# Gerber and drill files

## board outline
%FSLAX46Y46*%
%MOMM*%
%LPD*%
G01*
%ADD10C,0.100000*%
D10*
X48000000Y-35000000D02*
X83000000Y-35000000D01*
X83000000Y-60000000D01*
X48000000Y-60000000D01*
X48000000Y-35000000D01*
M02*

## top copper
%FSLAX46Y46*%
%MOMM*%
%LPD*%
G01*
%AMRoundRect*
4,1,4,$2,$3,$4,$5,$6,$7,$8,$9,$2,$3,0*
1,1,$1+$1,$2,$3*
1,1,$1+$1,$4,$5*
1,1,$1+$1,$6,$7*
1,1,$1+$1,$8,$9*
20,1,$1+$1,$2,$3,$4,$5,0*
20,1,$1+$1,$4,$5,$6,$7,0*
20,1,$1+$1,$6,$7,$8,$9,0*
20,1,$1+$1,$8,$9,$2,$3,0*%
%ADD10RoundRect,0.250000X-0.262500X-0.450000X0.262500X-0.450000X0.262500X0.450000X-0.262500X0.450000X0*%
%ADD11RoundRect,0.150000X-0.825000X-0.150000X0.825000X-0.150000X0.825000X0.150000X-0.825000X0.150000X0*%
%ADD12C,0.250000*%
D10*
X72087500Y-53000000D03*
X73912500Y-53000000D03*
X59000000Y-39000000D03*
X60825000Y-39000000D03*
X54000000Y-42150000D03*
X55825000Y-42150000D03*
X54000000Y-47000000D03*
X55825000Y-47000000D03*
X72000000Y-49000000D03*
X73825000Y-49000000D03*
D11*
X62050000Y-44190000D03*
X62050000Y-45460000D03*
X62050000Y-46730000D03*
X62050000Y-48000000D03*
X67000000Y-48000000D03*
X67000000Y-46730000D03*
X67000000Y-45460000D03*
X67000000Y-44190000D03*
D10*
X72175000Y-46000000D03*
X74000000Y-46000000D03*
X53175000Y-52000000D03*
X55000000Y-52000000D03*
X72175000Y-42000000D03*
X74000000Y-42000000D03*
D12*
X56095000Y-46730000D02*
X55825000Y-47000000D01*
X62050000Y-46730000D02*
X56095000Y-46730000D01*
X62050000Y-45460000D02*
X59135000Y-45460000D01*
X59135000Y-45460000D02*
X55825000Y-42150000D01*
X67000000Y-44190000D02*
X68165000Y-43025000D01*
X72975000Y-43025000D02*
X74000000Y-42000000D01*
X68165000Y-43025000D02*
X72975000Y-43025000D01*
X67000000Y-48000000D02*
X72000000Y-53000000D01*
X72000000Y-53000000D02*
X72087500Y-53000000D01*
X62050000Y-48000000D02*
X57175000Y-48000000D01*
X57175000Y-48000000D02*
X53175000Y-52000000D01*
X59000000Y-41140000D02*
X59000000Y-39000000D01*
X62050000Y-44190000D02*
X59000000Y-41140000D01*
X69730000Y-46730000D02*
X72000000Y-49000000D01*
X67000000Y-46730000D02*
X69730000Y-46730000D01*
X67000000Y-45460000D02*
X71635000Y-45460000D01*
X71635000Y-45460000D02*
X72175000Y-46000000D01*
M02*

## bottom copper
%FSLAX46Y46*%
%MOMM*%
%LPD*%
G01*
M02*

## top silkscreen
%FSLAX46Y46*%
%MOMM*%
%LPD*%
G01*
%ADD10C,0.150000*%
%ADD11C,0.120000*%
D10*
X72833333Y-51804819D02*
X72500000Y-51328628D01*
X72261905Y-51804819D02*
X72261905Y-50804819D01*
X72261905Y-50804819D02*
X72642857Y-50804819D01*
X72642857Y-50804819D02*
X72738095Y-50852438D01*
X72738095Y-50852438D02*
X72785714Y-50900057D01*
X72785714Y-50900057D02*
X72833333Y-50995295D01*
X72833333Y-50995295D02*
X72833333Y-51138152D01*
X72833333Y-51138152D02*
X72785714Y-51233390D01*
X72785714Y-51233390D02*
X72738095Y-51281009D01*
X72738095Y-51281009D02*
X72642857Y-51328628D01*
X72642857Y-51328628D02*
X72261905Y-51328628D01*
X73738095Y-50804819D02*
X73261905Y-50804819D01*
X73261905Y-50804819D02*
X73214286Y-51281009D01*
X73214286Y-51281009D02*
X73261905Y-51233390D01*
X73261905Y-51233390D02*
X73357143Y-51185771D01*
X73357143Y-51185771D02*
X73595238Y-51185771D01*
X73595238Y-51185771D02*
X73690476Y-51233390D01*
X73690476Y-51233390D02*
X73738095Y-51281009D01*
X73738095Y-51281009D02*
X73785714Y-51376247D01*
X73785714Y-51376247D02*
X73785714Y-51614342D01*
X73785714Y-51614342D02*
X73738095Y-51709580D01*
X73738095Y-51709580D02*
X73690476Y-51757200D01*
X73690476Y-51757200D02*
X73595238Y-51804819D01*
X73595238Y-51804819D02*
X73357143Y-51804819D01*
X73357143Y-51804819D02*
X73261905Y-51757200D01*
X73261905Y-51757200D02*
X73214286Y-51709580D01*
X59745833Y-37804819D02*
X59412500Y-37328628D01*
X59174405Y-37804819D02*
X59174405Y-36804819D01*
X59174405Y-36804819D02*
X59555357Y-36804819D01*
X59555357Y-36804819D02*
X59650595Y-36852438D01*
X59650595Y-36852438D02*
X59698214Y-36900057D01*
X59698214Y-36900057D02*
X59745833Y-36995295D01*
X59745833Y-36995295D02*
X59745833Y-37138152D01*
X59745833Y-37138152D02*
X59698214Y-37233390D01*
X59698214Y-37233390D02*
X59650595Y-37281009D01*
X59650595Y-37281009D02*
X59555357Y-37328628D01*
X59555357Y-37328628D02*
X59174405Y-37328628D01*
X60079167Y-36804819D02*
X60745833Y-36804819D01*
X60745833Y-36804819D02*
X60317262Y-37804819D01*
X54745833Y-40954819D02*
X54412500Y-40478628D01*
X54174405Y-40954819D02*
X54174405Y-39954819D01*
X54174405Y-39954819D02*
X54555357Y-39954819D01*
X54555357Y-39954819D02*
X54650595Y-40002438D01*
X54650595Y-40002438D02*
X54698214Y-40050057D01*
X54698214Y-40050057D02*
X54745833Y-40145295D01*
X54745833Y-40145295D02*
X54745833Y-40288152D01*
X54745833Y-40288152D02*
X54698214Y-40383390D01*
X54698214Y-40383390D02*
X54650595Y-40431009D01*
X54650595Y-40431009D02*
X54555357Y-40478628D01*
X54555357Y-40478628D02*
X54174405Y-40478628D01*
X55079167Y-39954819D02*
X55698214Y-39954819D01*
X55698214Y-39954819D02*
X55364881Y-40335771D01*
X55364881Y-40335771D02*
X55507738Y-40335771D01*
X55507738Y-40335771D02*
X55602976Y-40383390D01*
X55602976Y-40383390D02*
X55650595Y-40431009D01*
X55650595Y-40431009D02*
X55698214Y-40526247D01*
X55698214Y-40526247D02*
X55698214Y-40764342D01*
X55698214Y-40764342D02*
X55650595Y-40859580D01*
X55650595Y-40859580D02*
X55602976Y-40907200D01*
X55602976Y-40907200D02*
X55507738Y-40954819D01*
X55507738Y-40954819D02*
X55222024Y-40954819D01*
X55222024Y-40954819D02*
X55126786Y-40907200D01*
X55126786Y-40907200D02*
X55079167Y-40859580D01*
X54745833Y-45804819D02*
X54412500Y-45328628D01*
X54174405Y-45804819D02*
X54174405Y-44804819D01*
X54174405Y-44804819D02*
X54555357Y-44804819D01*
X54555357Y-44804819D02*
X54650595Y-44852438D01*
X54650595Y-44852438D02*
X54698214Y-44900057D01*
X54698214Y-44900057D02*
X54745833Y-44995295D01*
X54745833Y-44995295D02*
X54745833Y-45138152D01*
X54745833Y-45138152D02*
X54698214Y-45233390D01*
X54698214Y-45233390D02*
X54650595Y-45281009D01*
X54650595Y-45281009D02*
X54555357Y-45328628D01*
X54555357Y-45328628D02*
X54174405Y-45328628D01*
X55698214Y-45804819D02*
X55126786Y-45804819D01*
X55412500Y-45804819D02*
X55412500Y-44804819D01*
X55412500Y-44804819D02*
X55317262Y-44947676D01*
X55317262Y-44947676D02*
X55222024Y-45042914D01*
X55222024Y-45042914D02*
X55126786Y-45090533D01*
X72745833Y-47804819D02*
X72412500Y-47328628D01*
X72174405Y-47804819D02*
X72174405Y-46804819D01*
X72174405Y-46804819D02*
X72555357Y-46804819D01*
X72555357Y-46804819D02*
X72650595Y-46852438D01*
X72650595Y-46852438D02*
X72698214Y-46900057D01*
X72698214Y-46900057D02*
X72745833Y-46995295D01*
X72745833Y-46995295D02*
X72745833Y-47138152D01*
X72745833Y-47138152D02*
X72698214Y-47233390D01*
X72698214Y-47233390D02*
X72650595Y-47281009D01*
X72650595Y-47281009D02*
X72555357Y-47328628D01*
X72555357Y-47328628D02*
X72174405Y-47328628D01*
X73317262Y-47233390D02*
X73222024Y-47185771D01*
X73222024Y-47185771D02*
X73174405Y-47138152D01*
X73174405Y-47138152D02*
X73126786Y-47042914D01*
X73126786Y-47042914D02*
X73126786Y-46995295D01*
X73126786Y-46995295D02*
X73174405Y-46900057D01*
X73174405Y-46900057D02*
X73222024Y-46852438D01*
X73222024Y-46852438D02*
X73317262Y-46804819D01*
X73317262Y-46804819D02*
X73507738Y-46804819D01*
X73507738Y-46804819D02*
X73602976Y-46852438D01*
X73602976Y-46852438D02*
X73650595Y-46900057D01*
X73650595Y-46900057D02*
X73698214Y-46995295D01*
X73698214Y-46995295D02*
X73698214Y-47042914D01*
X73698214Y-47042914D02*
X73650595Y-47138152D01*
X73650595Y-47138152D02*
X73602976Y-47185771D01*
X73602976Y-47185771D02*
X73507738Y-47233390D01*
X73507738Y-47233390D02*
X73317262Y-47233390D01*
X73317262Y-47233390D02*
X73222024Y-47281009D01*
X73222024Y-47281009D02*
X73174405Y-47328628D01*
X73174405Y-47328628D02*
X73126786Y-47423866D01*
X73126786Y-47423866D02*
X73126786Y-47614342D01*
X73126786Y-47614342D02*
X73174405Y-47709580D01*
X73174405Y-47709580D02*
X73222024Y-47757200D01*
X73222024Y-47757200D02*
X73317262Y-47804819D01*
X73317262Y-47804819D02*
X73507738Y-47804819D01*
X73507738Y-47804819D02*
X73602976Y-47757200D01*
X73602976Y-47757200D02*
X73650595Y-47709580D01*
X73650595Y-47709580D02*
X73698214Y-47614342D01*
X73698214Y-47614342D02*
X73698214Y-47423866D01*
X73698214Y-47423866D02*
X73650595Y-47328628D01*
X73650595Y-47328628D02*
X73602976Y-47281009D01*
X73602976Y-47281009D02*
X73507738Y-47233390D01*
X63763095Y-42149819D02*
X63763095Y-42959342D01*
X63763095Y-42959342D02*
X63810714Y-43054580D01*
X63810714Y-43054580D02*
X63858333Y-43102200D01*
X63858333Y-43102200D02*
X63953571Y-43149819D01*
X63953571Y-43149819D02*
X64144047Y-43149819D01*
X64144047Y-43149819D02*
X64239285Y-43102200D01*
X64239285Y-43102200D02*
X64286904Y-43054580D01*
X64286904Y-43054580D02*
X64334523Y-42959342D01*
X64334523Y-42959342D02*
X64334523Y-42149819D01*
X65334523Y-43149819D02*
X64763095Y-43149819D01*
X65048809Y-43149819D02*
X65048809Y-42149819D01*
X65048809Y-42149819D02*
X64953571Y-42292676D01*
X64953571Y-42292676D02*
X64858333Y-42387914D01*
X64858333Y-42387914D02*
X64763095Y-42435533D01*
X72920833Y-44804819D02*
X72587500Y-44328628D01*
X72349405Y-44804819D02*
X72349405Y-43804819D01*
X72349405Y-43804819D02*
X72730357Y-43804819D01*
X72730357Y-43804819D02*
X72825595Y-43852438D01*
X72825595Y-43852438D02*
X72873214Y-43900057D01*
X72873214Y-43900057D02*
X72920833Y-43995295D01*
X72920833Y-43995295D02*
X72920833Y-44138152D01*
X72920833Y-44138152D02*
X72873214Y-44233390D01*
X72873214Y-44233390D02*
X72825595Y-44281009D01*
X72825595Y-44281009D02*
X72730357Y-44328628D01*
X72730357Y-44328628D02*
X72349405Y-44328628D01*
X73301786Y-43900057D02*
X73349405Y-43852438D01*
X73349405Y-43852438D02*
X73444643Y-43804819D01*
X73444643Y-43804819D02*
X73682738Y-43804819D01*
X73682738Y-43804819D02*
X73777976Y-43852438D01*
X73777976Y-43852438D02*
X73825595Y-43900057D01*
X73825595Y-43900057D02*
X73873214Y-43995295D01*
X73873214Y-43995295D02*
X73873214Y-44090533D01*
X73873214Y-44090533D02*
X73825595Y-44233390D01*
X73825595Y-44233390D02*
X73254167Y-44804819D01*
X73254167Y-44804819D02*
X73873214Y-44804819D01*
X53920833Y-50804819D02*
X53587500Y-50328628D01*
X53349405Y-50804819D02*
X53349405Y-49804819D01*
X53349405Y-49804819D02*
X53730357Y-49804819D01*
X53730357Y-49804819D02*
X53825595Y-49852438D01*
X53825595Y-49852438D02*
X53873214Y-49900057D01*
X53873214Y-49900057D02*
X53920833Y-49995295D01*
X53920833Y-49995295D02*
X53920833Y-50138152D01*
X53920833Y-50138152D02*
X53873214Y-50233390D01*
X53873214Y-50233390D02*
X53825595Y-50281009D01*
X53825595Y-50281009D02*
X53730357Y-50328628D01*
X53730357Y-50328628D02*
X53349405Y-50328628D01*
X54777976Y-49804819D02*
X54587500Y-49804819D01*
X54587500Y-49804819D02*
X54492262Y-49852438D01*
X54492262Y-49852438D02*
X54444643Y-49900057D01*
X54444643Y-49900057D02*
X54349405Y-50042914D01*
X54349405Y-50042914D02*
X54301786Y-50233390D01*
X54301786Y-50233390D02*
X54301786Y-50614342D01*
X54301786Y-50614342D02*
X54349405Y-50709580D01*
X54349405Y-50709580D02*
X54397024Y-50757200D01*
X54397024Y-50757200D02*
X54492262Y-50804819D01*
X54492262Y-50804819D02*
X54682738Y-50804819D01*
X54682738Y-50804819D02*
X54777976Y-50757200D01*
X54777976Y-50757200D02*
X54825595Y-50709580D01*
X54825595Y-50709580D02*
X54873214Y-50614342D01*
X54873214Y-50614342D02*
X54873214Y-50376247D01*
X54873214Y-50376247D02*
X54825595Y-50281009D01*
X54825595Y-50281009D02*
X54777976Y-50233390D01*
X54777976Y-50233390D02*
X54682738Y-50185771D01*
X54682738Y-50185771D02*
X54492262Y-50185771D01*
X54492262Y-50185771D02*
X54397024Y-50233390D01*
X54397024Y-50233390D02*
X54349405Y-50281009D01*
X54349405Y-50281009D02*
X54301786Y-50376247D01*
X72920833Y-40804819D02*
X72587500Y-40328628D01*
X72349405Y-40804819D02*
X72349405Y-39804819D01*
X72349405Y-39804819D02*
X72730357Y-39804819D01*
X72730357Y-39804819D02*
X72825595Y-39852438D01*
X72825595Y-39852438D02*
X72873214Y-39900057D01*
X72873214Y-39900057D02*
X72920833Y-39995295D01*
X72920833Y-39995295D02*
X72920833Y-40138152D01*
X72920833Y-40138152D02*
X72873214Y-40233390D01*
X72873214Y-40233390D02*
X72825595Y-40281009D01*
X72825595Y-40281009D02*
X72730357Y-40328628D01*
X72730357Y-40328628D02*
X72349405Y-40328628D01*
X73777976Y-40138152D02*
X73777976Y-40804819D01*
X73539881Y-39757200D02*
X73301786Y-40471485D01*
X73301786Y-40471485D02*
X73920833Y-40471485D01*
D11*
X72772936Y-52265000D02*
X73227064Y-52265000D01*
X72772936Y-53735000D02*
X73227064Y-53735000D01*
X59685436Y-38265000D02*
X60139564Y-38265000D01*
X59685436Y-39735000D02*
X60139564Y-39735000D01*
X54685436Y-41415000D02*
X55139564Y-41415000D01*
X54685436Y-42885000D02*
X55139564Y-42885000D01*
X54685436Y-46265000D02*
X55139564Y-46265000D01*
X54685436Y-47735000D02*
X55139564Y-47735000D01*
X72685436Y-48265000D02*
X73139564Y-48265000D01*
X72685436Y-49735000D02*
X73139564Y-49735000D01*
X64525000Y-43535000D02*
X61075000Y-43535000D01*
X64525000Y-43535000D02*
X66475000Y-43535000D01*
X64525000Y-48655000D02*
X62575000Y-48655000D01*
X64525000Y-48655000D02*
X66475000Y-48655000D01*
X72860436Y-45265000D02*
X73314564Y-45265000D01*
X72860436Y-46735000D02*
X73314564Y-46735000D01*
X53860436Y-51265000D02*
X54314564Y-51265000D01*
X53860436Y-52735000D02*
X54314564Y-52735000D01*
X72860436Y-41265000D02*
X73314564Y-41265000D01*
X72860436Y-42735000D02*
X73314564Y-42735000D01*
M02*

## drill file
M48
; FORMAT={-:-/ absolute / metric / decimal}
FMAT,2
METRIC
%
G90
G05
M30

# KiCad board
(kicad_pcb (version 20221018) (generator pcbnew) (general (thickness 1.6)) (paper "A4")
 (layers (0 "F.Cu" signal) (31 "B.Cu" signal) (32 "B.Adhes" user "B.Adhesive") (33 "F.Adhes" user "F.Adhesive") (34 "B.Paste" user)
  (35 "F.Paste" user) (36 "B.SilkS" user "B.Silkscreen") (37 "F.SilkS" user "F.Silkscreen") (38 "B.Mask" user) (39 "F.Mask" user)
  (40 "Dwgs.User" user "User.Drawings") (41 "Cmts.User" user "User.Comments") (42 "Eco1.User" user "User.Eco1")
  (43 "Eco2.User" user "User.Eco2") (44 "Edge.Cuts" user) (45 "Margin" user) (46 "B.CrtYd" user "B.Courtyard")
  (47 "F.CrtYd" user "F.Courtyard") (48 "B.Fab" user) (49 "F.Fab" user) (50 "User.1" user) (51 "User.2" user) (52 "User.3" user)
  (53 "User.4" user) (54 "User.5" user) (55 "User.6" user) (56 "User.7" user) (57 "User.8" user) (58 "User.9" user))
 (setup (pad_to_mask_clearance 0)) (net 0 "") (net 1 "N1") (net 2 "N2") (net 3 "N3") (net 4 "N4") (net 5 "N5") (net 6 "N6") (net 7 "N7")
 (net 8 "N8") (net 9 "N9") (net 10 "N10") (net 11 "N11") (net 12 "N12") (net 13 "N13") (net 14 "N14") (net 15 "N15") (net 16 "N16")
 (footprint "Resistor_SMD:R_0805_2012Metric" (layer "F.Cu") (at 73 53)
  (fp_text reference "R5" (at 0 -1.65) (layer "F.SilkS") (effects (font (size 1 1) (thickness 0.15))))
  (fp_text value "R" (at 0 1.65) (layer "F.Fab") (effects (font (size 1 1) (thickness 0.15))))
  (fp_line (start -0.227064 -0.735) (end 0.227064 -0.735) (stroke (width 0.12) (type solid)) (layer "F.SilkS"))
  (fp_line (start -0.227064 0.735) (end 0.227064 0.735) (stroke (width 0.12) (type solid)) (layer "F.SilkS"))
  (pad "1" smd roundrect (at -0.9125 0) (size 1.025 1.4) (layers "F.Cu" "F.Paste" "F.Mask") (roundrect_rratio 0.243902) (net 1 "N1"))
  (pad "2" smd roundrect (at 0.9125 0) (size 1.025 1.4) (layers "F.Cu" "F.Paste" "F.Mask") (roundrect_rratio 0.243902) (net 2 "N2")))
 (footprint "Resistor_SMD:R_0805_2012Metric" (layer "F.Cu") (at 59.9125 39)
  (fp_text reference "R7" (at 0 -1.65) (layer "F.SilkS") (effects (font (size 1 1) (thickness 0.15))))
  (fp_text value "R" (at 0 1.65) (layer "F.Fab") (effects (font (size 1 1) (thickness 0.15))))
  (fp_line (start -0.227064 -0.735) (end 0.227064 -0.735) (stroke (width 0.12) (type solid)) (layer "F.SilkS"))
  (fp_line (start -0.227064 0.735) (end 0.227064 0.735) (stroke (width 0.12) (type solid)) (layer "F.SilkS"))
  (pad "1" smd roundrect (at -0.9125 0) (size 1.025 1.4) (layers "F.Cu" "F.Paste" "F.Mask") (roundrect_rratio 0.243902) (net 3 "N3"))
  (pad "2" smd roundrect (at 0.9125 0) (size 1.025 1.4) (layers "F.Cu" "F.Paste" "F.Mask") (roundrect_rratio 0.243902) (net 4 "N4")))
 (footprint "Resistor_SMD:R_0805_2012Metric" (layer "F.Cu") (at 54.9125 42.15)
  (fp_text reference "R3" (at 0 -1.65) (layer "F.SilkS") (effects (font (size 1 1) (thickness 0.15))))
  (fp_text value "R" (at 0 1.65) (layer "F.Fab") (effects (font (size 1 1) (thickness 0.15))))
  (fp_line (start -0.227064 -0.735) (end 0.227064 -0.735) (stroke (width 0.12) (type solid)) (layer "F.SilkS"))
  (fp_line (start -0.227064 0.735) (end 0.227064 0.735) (stroke (width 0.12) (type solid)) (layer "F.SilkS"))
  (pad "1" smd roundrect (at -0.9125 0) (size 1.025 1.4) (layers "F.Cu" "F.Paste" "F.Mask") (roundrect_rratio 0.243902) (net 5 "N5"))
  (pad "2" smd roundrect (at 0.9125 0) (size 1.025 1.4) (layers "F.Cu" "F.Paste" "F.Mask") (roundrect_rratio 0.243902) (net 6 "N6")))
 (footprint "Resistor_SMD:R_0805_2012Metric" (layer "F.Cu") (at 54.9125 47)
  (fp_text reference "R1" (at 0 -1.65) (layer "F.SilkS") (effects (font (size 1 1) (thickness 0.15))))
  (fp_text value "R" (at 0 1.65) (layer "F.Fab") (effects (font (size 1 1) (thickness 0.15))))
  (fp_line (start -0.227064 -0.735) (end 0.227064 -0.735) (stroke (width 0.12) (type solid)) (layer "F.SilkS"))
  (fp_line (start -0.227064 0.735) (end 0.227064 0.735) (stroke (width 0.12) (type solid)) (layer "F.SilkS"))
  (pad "1" smd roundrect (at -0.9125 0) (size 1.025 1.4) (layers "F.Cu" "F.Paste" "F.Mask") (roundrect_rratio 0.243902) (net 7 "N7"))
  (pad "2" smd roundrect (at 0.9125 0) (size 1.025 1.4) (layers "F.Cu" "F.Paste" "F.Mask") (roundrect_rratio 0.243902) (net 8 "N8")))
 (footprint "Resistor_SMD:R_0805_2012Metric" (layer "F.Cu") (at 72.9125 49)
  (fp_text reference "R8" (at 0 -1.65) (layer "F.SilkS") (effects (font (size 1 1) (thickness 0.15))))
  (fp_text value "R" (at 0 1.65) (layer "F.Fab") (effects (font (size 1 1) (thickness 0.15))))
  (fp_line (start -0.227064 -0.735) (end 0.227064 -0.735) (stroke (width 0.12) (type solid)) (layer "F.SilkS"))
  (fp_line (start -0.227064 0.735) (end 0.227064 0.735) (stroke (width 0.12) (type solid)) (layer "F.SilkS"))
  (pad "1" smd roundrect (at -0.9125 0) (size 1.025 1.4) (layers "F.Cu" "F.Paste" "F.Mask") (roundrect_rratio 0.243902) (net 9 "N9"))
  (pad "2" smd roundrect (at 0.9125 0) (size 1.025 1.4) (layers "F.Cu" "F.Paste" "F.Mask") (roundrect_rratio 0.243902) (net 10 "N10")))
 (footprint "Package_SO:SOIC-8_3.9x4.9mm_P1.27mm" (layer "F.Cu") (at 64.525 46.095)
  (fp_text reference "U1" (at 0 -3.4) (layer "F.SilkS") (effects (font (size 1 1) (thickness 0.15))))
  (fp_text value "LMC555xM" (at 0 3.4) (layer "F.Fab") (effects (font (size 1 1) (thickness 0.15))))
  (fp_line (start 0 -2.56) (end -3.45 -2.56) (stroke (width 0.12) (type solid)) (layer "F.SilkS"))
  (fp_line (start 0 -2.56) (end 1.95 -2.56) (stroke (width 0.12) (type solid)) (layer "F.SilkS"))
  (fp_line (start 0 2.56) (end -1.95 2.56) (stroke (width 0.12) (type solid)) (layer "F.SilkS"))
  (fp_line (start 0 2.56) (end 1.95 2.56) (stroke (width 0.12) (type solid)) (layer "F.SilkS"))
  (pad "1" smd roundrect (at -2.475 -1.905) (size 1.95 0.6) (layers "F.Cu" "F.Paste" "F.Mask") (roundrect_rratio 0.25) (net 3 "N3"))
  (pad "2" smd roundrect (at -2.475 -0.635) (size 1.95 0.6) (layers "F.Cu" "F.Paste" "F.Mask") (roundrect_rratio 0.25) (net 6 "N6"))
  (pad "3" smd roundrect (at -2.475 0.635) (size 1.95 0.6) (layers "F.Cu" "F.Paste" "F.Mask") (roundrect_rratio 0.25) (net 8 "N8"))
  (pad "4" smd roundrect (at -2.475 1.905) (size 1.95 0.6) (layers "F.Cu" "F.Paste" "F.Mask") (roundrect_rratio 0.25) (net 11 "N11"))
  (pad "5" smd roundrect (at 2.475 1.905) (size 1.95 0.6) (layers "F.Cu" "F.Paste" "F.Mask") (roundrect_rratio 0.25) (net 1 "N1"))
  (pad "6" smd roundrect (at 2.475 0.635) (size 1.95 0.6) (layers "F.Cu" "F.Paste" "F.Mask") (roundrect_rratio 0.25) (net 9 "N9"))
  (pad "7" smd roundrect (at 2.475 -0.635) (size 1.95 0.6) (layers "F.Cu" "F.Paste" "F.Mask") (roundrect_rratio 0.25) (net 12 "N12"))
  (pad "8" smd roundrect (at 2.475 -1.905) (size 1.95 0.6) (layers "F.Cu" "F.Paste" "F.Mask") (roundrect_rratio 0.25) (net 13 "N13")))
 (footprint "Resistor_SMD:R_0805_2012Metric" (layer "F.Cu") (at 73.0875 46)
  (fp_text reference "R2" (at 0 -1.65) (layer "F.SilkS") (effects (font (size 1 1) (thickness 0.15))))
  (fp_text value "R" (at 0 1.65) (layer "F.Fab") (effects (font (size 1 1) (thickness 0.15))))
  (fp_line (start -0.227064 -0.735) (end 0.227064 -0.735) (stroke (width 0.12) (type solid)) (layer "F.SilkS"))
  (fp_line (start -0.227064 0.735) (end 0.227064 0.735) (stroke (width 0.12) (type solid)) (layer "F.SilkS"))
  (pad "1" smd roundrect (at -0.9125 0) (size 1.025 1.4) (layers "F.Cu" "F.Paste" "F.Mask") (roundrect_rratio 0.243902) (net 12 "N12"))
  (pad "2" smd roundrect (at 0.9125 0) (size 1.025 1.4) (layers "F.Cu" "F.Paste" "F.Mask") (roundrect_rratio 0.243902) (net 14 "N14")))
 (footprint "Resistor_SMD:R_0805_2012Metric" (layer "F.Cu") (at 54.0875 52)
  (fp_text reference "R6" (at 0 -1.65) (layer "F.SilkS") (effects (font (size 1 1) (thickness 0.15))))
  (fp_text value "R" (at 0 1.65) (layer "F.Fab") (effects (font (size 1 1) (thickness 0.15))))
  (fp_line (start -0.227064 -0.735) (end 0.227064 -0.735) (stroke (width 0.12) (type solid)) (layer "F.SilkS"))
  (fp_line (start -0.227064 0.735) (end 0.227064 0.735) (stroke (width 0.12) (type solid)) (layer "F.SilkS"))
  (pad "1" smd roundrect (at -0.9125 0) (size 1.025 1.4) (layers "F.Cu" "F.Paste" "F.Mask") (roundrect_rratio 0.243902) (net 11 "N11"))
  (pad "2" smd roundrect (at 0.9125 0) (size 1.025 1.4) (layers "F.Cu" "F.Paste" "F.Mask") (roundrect_rratio 0.243902) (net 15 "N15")))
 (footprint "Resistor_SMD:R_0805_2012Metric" (layer "F.Cu") (at 73.0875 42)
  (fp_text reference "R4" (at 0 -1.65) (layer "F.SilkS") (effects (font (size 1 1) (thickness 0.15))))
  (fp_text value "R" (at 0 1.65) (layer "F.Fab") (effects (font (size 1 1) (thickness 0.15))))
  (fp_line (start -0.227064 -0.735) (end 0.227064 -0.735) (stroke (width 0.12) (type solid)) (layer "F.SilkS"))
  (fp_line (start -0.227064 0.735) (end 0.227064 0.735) (stroke (width 0.12) (type solid)) (layer "F.SilkS"))
  (pad "1" smd roundrect (at -0.9125 0) (size 1.025 1.4) (layers "F.Cu" "F.Paste" "F.Mask") (roundrect_rratio 0.243902) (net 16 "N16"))
  (pad "2" smd roundrect (at 0.9125 0) (size 1.025 1.4) (layers "F.Cu" "F.Paste" "F.Mask") (roundrect_rratio 0.243902) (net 13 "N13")))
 (gr_rect (start 48 35) (end 83 60) (stroke (width 0.1) (type default)) (fill none) (layer "Edge.Cuts"))
 (segment (start 56.095 46.73) (end 55.825 47) (width 0.25) (layer "F.Cu") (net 8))
 (segment (start 62.05 46.73) (end 56.095 46.73) (width 0.25) (layer "F.Cu") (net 8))
 (segment (start 62.05 45.46) (end 59.135 45.46) (width 0.25) (layer "F.Cu") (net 6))
 (segment (start 59.135 45.46) (end 55.825 42.15) (width 0.25) (layer "F.Cu") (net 6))
 (segment (start 67 44.19) (end 68.165 43.025) (width 0.25) (layer "F.Cu") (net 13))
 (segment (start 72.975 43.025) (end 74 42) (width 0.25) (layer "F.Cu") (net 13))
 (segment (start 68.165 43.025) (end 72.975 43.025) (width 0.25) (layer "F.Cu") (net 13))
 (segment (start 67 48) (end 72 53) (width 0.25) (layer "F.Cu") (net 1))
 (segment (start 72 53) (end 72.0875 53) (width 0.25) (layer "F.Cu") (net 1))
 (segment (start 62.05 48) (end 57.175 48) (width 0.25) (layer "F.Cu") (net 11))
 (segment (start 57.175 48) (end 53.175 52) (width 0.25) (layer "F.Cu") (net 11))
 (segment (start 59 41.14) (end 59 39) (width 0.25) (layer "F.Cu") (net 3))
 (segment (start 62.05 44.19) (end 59 41.14) (width 0.25) (layer "F.Cu") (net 3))
 (segment (start 69.73 46.73) (end 72 49) (width 0.25) (layer "F.Cu") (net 9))
 (segment (start 67 46.73) (end 69.73 46.73) (width 0.25) (layer "F.Cu") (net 9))
 (segment (start 67 45.46) (end 71.635 45.46) (width 0.25) (layer "F.Cu") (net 12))
 (segment (start 71.635 45.46) (end 72.175 46) (width 0.25) (layer "F.Cu") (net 12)))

